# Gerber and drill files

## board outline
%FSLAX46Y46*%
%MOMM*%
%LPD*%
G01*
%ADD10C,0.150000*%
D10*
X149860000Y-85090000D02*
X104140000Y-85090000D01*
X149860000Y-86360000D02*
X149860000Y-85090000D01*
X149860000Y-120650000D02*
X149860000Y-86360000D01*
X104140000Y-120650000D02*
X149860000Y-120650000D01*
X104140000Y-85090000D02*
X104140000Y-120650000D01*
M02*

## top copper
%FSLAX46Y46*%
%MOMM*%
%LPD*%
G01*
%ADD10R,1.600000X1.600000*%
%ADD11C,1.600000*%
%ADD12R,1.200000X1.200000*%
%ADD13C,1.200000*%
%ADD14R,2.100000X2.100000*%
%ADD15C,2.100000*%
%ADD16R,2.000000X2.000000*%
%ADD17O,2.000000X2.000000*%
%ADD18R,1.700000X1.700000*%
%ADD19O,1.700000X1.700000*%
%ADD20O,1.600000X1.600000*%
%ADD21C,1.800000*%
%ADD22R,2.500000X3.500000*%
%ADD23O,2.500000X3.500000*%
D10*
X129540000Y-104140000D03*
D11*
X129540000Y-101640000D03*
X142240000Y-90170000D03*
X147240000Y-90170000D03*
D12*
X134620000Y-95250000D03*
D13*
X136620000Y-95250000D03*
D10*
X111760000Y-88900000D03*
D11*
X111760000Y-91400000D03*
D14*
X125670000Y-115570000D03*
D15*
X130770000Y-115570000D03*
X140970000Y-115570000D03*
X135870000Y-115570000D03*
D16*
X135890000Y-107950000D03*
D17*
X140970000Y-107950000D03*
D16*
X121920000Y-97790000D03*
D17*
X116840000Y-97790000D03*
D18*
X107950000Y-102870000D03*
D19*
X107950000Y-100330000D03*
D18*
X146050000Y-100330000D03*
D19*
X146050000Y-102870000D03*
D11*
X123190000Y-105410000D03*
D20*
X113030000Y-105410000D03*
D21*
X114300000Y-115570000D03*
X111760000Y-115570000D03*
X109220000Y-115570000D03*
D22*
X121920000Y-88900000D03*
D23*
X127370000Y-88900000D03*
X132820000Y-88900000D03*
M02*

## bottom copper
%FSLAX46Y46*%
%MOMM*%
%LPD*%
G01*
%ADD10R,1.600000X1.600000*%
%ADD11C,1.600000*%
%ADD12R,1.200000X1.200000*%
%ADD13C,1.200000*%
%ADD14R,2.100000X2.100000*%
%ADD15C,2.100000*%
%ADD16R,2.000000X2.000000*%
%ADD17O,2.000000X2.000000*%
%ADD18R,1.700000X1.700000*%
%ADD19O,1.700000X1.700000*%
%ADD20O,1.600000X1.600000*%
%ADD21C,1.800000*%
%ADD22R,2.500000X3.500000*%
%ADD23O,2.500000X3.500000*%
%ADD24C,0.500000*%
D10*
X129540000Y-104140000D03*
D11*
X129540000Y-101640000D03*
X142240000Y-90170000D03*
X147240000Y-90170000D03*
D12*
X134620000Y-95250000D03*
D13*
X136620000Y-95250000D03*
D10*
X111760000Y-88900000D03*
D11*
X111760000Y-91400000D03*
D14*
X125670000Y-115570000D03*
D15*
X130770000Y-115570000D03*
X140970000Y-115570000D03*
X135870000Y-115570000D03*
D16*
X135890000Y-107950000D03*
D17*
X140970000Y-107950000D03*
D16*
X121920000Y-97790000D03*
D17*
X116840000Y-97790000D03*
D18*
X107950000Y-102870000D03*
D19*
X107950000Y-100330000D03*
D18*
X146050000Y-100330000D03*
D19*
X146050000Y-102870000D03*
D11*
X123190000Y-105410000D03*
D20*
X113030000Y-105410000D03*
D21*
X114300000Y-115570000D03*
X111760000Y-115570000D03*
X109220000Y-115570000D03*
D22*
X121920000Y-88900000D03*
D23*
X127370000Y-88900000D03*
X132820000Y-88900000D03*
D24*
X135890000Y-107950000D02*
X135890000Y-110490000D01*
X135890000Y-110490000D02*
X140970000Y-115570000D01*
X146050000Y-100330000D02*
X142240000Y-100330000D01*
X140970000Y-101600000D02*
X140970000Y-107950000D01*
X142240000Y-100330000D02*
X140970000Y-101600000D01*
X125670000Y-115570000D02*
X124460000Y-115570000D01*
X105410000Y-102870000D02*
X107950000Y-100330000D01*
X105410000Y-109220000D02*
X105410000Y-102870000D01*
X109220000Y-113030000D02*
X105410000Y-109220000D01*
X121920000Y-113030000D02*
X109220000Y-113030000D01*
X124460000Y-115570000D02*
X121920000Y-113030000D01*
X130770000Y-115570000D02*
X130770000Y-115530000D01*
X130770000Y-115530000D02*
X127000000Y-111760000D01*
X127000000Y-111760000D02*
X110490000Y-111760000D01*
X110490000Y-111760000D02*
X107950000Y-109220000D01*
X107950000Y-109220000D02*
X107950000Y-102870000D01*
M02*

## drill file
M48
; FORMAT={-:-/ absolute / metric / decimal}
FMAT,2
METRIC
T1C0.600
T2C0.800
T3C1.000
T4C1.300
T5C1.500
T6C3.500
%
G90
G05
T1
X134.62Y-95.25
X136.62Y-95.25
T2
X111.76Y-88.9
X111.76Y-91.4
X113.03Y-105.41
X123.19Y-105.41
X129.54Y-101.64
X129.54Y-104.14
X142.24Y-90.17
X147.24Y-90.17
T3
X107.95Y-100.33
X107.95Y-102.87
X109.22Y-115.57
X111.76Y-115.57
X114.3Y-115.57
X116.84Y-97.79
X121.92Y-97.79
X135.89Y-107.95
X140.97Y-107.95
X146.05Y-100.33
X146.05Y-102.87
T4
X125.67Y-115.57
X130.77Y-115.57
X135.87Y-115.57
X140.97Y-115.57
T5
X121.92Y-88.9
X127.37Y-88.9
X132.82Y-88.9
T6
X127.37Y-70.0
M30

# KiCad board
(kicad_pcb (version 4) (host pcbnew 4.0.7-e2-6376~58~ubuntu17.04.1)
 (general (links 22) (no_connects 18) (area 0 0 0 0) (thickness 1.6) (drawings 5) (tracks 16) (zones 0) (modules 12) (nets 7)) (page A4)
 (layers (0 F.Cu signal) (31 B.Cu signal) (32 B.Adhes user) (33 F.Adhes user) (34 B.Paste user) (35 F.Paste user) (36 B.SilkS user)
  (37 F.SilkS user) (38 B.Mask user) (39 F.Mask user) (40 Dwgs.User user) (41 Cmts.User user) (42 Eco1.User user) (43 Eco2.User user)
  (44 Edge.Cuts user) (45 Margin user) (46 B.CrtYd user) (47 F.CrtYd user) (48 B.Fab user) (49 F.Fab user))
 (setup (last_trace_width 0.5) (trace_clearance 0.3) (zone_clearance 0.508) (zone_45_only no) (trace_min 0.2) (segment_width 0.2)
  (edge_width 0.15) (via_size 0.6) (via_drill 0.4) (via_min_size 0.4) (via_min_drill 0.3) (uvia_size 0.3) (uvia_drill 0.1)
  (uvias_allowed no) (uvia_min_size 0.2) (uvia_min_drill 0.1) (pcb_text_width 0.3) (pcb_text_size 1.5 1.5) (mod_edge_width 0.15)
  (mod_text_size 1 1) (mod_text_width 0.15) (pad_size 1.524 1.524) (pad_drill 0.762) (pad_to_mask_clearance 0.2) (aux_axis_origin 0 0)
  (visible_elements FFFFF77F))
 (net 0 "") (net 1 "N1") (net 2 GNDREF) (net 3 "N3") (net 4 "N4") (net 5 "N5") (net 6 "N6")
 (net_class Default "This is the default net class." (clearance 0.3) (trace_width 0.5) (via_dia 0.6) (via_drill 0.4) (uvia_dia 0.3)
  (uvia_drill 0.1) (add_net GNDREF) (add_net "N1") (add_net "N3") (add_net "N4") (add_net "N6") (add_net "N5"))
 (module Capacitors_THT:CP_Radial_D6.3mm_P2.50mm (layer F.Cu) (at 129.54 104.14 90)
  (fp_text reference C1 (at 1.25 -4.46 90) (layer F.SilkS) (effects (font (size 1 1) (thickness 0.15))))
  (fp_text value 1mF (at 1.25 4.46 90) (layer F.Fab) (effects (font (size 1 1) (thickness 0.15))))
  (pad 1 thru_hole rect (at 0 0 90) (size 1.6 1.6) (drill 0.8) (layers *.Cu *.Mask) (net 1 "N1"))
  (pad 2 thru_hole circle (at 2.5 0 90) (size 1.6 1.6) (drill 0.8) (layers *.Cu *.Mask) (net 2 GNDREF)))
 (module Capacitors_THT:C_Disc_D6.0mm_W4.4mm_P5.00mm (layer F.Cu) (at 142.24 90.17)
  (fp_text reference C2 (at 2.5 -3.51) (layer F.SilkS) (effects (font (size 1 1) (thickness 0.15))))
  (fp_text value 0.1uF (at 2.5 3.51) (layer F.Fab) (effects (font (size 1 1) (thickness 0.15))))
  (pad 1 thru_hole circle (at 0 0) (size 1.6 1.6) (drill 0.8) (layers *.Cu *.Mask) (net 1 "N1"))
  (pad 2 thru_hole circle (at 5 0) (size 1.6 1.6) (drill 0.8) (layers *.Cu *.Mask) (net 2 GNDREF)))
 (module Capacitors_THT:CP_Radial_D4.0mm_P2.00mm (layer F.Cu) (at 134.62 95.25)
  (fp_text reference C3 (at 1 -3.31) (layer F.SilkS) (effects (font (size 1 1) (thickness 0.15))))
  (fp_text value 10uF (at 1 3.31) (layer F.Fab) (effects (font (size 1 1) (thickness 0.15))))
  (pad 1 thru_hole rect (at 0 0) (size 1.2 1.2) (drill 0.6) (layers *.Cu *.Mask) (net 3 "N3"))
  (pad 2 thru_hole circle (at 2 0) (size 1.2 1.2) (drill 0.6) (layers *.Cu *.Mask) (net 2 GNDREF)))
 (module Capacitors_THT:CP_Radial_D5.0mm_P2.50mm (layer F.Cu) (at 111.76 88.9 270)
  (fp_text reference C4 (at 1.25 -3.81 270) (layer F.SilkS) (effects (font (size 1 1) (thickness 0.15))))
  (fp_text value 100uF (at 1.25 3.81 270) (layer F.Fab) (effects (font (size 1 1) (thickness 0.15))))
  (pad 1 thru_hole rect (at 0 0 270) (size 1.6 1.6) (drill 0.8) (layers *.Cu *.Mask) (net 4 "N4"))
  (pad 2 thru_hole circle (at 2.5 0 270) (size 1.6 1.6) (drill 0.8) (layers *.Cu *.Mask) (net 2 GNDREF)))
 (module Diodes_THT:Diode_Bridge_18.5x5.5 (layer F.Cu) (at 140.97 115.57)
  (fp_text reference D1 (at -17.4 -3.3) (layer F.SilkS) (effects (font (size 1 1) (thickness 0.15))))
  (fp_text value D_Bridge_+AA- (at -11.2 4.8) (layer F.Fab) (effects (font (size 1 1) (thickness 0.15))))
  (pad 3 thru_hole rect (at -15.3 0) (size 2.1 2.1) (drill 1.3) (layers *.Cu *.Mask) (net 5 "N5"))
  (pad 2 thru_hole circle (at -10.2 0) (size 2.1 2.1) (drill 1.3) (layers *.Cu *.Mask) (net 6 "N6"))
  (pad 1 thru_hole circle (at 0 0) (size 2.1 2.1) (drill 1.3) (layers *.Cu *.Mask) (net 1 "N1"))
  (pad 4 thru_hole circle (at -5.1 0) (size 2.1 2.1) (drill 1.3) (layers *.Cu *.Mask) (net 2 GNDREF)))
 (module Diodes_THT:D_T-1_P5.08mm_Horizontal (layer F.Cu) (at 135.89 107.95)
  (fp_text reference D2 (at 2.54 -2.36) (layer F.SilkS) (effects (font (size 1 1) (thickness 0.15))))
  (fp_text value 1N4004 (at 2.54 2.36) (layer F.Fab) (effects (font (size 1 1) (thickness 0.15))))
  (pad 1 thru_hole rect (at 0 0) (size 2 2) (drill 1) (layers *.Cu *.Mask) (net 1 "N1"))
  (pad 2 thru_hole oval (at 5.08 0) (size 2 2) (drill 1) (layers *.Cu *.Mask) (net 4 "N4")))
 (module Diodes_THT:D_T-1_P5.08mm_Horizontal (layer F.Cu) (at 121.92 97.79 180)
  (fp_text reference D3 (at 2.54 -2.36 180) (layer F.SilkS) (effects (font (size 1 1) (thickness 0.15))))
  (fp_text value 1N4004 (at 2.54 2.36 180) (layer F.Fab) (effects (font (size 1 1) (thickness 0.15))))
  (pad 1 thru_hole rect (at 0 0 180) (size 2 2) (drill 1) (layers *.Cu *.Mask) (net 4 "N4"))
  (pad 2 thru_hole oval (at 5.08 0 180) (size 2 2) (drill 1) (layers *.Cu *.Mask) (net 3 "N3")))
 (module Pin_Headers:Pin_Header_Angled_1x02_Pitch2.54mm (layer F.Cu) (at 107.95 102.87 180)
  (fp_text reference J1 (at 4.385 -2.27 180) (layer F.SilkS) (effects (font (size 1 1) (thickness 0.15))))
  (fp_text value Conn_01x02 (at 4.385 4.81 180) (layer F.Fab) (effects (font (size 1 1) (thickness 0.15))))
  (pad 1 thru_hole rect (at 0 0 180) (size 1.7 1.7) (drill 1) (layers *.Cu *.Mask) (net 6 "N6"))
  (pad 2 thru_hole oval (at 0 2.54 180) (size 1.7 1.7) (drill 1) (layers *.Cu *.Mask) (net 5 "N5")))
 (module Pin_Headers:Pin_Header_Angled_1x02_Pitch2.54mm (layer F.Cu) (at 146.05 100.33)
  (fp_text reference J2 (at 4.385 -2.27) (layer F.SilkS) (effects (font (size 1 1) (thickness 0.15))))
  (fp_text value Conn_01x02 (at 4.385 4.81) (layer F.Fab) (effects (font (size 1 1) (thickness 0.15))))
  (pad 1 thru_hole rect (at 0 0) (size 1.7 1.7) (drill 1) (layers *.Cu *.Mask) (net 4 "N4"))
  (pad 2 thru_hole oval (at 0 2.54) (size 1.7 1.7) (drill 1) (layers *.Cu *.Mask) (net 2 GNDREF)))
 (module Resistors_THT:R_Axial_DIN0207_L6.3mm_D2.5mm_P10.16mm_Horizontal (layer F.Cu) (at 123.19 105.41 180)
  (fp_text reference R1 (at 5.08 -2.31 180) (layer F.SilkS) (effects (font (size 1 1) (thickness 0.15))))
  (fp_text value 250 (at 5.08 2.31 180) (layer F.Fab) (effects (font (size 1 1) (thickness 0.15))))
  (pad 1 thru_hole circle (at 0 0 180) (size 1.6 1.6) (drill 0.8) (layers *.Cu *.Mask) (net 4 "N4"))
  (pad 2 thru_hole oval (at 10.16 0 180) (size 1.6 1.6) (drill 0.8) (layers *.Cu *.Mask) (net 3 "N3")))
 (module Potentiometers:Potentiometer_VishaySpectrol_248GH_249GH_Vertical (layer F.Cu) (at 109.22 115.57 270)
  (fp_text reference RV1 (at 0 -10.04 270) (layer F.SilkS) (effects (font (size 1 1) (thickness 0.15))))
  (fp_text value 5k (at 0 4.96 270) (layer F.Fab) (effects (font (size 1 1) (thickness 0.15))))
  (pad 3 thru_hole circle (at 0 -5.08 270) (size 1.8 1.8) (drill 1) (layers *.Cu *.Mask) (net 2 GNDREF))
  (pad 2 thru_hole circle (at 0 -2.54 270) (size 1.8 1.8) (drill 1) (layers *.Cu *.Mask) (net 2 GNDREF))
  (pad 1 thru_hole circle (at 0 0 270) (size 1.8 1.8) (drill 1) (layers *.Cu *.Mask) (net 3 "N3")))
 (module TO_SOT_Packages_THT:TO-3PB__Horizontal (layer F.Cu) (at 121.92 88.9)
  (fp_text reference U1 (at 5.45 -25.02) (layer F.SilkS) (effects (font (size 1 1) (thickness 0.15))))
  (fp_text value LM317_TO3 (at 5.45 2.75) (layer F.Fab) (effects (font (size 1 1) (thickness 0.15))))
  (pad 0 np_thru_hole oval (at 5.45 -18.9) (size 3.5 3.5) (drill 3.5) (layers *.Cu *.Mask))
  (pad 1 thru_hole rect (at 0 0) (size 2.5 3.5) (drill 1.5) (layers *.Cu *.Mask) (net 3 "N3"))
  (pad 2 thru_hole oval (at 5.45 0) (size 2.5 3.5) (drill 1.5) (layers *.Cu *.Mask) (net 4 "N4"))
  (pad 3 thru_hole oval (at 10.9 0) (size 2.5 3.5) (drill 1.5) (layers *.Cu *.Mask) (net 1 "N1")))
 (gr_line (start 149.86 85.09) (end 104.14 85.09) (angle 90) (layer Edge.Cuts) (width 0.15))
 (gr_line (start 149.86 86.36) (end 149.86 85.09) (angle 90) (layer Edge.Cuts) (width 0.15))
 (gr_line (start 149.86 120.65) (end 149.86 86.36) (angle 90) (layer Edge.Cuts) (width 0.15))
 (gr_line (start 104.14 120.65) (end 149.86 120.65) (angle 90) (layer Edge.Cuts) (width 0.15))
 (gr_line (start 104.14 85.09) (end 104.14 120.65) (angle 90) (layer Edge.Cuts) (width 0.15))
 (segment (start 135.89 107.95) (end 135.89 110.49) (width 0.5) (layer B.Cu) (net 1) (status 400000))
 (segment (start 135.89 110.49) (end 140.97 115.57) (width 0.5) (layer B.Cu) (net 1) (status 800000))
 (segment (start 146.05 100.33) (end 142.24 100.33) (width 0.5) (layer B.Cu) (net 4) (status 400000))
 (segment (start 140.97 101.6) (end 140.97 107.95) (width 0.5) (layer B.Cu) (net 4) (status 800000))
 (segment (start 142.24 100.33) (end 140.97 101.6) (width 0.5) (layer B.Cu) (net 4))
 (segment (start 125.67 115.57) (end 124.46 115.57) (width 0.5) (layer B.Cu) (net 5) (status 400000))
 (segment (start 105.41 102.87) (end 107.95 100.33) (width 0.5) (layer B.Cu) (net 5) (status 800000))
 (segment (start 105.41 109.22) (end 105.41 102.87) (width 0.5) (layer B.Cu) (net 5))
 (segment (start 109.22 113.03) (end 105.41 109.22) (width 0.5) (layer B.Cu) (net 5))
 (segment (start 121.92 113.03) (end 109.22 113.03) (width 0.5) (layer B.Cu) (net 5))
 (segment (start 124.46 115.57) (end 121.92 113.03) (width 0.5) (layer B.Cu) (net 5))
 (segment (start 130.77 115.57) (end 130.77 115.53) (width 0.5) (layer B.Cu) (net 6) (status C00000))
 (segment (start 130.77 115.53) (end 127 111.76) (width 0.5) (layer B.Cu) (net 6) (status 400000))
 (segment (start 127 111.76) (end 110.49 111.76) (width 0.5) (layer B.Cu) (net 6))
 (segment (start 110.49 111.76) (end 107.95 109.22) (width 0.5) (layer B.Cu) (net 6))
 (segment (start 107.95 109.22) (end 107.95 102.87) (width 0.5) (layer B.Cu) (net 6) (status 800000)))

